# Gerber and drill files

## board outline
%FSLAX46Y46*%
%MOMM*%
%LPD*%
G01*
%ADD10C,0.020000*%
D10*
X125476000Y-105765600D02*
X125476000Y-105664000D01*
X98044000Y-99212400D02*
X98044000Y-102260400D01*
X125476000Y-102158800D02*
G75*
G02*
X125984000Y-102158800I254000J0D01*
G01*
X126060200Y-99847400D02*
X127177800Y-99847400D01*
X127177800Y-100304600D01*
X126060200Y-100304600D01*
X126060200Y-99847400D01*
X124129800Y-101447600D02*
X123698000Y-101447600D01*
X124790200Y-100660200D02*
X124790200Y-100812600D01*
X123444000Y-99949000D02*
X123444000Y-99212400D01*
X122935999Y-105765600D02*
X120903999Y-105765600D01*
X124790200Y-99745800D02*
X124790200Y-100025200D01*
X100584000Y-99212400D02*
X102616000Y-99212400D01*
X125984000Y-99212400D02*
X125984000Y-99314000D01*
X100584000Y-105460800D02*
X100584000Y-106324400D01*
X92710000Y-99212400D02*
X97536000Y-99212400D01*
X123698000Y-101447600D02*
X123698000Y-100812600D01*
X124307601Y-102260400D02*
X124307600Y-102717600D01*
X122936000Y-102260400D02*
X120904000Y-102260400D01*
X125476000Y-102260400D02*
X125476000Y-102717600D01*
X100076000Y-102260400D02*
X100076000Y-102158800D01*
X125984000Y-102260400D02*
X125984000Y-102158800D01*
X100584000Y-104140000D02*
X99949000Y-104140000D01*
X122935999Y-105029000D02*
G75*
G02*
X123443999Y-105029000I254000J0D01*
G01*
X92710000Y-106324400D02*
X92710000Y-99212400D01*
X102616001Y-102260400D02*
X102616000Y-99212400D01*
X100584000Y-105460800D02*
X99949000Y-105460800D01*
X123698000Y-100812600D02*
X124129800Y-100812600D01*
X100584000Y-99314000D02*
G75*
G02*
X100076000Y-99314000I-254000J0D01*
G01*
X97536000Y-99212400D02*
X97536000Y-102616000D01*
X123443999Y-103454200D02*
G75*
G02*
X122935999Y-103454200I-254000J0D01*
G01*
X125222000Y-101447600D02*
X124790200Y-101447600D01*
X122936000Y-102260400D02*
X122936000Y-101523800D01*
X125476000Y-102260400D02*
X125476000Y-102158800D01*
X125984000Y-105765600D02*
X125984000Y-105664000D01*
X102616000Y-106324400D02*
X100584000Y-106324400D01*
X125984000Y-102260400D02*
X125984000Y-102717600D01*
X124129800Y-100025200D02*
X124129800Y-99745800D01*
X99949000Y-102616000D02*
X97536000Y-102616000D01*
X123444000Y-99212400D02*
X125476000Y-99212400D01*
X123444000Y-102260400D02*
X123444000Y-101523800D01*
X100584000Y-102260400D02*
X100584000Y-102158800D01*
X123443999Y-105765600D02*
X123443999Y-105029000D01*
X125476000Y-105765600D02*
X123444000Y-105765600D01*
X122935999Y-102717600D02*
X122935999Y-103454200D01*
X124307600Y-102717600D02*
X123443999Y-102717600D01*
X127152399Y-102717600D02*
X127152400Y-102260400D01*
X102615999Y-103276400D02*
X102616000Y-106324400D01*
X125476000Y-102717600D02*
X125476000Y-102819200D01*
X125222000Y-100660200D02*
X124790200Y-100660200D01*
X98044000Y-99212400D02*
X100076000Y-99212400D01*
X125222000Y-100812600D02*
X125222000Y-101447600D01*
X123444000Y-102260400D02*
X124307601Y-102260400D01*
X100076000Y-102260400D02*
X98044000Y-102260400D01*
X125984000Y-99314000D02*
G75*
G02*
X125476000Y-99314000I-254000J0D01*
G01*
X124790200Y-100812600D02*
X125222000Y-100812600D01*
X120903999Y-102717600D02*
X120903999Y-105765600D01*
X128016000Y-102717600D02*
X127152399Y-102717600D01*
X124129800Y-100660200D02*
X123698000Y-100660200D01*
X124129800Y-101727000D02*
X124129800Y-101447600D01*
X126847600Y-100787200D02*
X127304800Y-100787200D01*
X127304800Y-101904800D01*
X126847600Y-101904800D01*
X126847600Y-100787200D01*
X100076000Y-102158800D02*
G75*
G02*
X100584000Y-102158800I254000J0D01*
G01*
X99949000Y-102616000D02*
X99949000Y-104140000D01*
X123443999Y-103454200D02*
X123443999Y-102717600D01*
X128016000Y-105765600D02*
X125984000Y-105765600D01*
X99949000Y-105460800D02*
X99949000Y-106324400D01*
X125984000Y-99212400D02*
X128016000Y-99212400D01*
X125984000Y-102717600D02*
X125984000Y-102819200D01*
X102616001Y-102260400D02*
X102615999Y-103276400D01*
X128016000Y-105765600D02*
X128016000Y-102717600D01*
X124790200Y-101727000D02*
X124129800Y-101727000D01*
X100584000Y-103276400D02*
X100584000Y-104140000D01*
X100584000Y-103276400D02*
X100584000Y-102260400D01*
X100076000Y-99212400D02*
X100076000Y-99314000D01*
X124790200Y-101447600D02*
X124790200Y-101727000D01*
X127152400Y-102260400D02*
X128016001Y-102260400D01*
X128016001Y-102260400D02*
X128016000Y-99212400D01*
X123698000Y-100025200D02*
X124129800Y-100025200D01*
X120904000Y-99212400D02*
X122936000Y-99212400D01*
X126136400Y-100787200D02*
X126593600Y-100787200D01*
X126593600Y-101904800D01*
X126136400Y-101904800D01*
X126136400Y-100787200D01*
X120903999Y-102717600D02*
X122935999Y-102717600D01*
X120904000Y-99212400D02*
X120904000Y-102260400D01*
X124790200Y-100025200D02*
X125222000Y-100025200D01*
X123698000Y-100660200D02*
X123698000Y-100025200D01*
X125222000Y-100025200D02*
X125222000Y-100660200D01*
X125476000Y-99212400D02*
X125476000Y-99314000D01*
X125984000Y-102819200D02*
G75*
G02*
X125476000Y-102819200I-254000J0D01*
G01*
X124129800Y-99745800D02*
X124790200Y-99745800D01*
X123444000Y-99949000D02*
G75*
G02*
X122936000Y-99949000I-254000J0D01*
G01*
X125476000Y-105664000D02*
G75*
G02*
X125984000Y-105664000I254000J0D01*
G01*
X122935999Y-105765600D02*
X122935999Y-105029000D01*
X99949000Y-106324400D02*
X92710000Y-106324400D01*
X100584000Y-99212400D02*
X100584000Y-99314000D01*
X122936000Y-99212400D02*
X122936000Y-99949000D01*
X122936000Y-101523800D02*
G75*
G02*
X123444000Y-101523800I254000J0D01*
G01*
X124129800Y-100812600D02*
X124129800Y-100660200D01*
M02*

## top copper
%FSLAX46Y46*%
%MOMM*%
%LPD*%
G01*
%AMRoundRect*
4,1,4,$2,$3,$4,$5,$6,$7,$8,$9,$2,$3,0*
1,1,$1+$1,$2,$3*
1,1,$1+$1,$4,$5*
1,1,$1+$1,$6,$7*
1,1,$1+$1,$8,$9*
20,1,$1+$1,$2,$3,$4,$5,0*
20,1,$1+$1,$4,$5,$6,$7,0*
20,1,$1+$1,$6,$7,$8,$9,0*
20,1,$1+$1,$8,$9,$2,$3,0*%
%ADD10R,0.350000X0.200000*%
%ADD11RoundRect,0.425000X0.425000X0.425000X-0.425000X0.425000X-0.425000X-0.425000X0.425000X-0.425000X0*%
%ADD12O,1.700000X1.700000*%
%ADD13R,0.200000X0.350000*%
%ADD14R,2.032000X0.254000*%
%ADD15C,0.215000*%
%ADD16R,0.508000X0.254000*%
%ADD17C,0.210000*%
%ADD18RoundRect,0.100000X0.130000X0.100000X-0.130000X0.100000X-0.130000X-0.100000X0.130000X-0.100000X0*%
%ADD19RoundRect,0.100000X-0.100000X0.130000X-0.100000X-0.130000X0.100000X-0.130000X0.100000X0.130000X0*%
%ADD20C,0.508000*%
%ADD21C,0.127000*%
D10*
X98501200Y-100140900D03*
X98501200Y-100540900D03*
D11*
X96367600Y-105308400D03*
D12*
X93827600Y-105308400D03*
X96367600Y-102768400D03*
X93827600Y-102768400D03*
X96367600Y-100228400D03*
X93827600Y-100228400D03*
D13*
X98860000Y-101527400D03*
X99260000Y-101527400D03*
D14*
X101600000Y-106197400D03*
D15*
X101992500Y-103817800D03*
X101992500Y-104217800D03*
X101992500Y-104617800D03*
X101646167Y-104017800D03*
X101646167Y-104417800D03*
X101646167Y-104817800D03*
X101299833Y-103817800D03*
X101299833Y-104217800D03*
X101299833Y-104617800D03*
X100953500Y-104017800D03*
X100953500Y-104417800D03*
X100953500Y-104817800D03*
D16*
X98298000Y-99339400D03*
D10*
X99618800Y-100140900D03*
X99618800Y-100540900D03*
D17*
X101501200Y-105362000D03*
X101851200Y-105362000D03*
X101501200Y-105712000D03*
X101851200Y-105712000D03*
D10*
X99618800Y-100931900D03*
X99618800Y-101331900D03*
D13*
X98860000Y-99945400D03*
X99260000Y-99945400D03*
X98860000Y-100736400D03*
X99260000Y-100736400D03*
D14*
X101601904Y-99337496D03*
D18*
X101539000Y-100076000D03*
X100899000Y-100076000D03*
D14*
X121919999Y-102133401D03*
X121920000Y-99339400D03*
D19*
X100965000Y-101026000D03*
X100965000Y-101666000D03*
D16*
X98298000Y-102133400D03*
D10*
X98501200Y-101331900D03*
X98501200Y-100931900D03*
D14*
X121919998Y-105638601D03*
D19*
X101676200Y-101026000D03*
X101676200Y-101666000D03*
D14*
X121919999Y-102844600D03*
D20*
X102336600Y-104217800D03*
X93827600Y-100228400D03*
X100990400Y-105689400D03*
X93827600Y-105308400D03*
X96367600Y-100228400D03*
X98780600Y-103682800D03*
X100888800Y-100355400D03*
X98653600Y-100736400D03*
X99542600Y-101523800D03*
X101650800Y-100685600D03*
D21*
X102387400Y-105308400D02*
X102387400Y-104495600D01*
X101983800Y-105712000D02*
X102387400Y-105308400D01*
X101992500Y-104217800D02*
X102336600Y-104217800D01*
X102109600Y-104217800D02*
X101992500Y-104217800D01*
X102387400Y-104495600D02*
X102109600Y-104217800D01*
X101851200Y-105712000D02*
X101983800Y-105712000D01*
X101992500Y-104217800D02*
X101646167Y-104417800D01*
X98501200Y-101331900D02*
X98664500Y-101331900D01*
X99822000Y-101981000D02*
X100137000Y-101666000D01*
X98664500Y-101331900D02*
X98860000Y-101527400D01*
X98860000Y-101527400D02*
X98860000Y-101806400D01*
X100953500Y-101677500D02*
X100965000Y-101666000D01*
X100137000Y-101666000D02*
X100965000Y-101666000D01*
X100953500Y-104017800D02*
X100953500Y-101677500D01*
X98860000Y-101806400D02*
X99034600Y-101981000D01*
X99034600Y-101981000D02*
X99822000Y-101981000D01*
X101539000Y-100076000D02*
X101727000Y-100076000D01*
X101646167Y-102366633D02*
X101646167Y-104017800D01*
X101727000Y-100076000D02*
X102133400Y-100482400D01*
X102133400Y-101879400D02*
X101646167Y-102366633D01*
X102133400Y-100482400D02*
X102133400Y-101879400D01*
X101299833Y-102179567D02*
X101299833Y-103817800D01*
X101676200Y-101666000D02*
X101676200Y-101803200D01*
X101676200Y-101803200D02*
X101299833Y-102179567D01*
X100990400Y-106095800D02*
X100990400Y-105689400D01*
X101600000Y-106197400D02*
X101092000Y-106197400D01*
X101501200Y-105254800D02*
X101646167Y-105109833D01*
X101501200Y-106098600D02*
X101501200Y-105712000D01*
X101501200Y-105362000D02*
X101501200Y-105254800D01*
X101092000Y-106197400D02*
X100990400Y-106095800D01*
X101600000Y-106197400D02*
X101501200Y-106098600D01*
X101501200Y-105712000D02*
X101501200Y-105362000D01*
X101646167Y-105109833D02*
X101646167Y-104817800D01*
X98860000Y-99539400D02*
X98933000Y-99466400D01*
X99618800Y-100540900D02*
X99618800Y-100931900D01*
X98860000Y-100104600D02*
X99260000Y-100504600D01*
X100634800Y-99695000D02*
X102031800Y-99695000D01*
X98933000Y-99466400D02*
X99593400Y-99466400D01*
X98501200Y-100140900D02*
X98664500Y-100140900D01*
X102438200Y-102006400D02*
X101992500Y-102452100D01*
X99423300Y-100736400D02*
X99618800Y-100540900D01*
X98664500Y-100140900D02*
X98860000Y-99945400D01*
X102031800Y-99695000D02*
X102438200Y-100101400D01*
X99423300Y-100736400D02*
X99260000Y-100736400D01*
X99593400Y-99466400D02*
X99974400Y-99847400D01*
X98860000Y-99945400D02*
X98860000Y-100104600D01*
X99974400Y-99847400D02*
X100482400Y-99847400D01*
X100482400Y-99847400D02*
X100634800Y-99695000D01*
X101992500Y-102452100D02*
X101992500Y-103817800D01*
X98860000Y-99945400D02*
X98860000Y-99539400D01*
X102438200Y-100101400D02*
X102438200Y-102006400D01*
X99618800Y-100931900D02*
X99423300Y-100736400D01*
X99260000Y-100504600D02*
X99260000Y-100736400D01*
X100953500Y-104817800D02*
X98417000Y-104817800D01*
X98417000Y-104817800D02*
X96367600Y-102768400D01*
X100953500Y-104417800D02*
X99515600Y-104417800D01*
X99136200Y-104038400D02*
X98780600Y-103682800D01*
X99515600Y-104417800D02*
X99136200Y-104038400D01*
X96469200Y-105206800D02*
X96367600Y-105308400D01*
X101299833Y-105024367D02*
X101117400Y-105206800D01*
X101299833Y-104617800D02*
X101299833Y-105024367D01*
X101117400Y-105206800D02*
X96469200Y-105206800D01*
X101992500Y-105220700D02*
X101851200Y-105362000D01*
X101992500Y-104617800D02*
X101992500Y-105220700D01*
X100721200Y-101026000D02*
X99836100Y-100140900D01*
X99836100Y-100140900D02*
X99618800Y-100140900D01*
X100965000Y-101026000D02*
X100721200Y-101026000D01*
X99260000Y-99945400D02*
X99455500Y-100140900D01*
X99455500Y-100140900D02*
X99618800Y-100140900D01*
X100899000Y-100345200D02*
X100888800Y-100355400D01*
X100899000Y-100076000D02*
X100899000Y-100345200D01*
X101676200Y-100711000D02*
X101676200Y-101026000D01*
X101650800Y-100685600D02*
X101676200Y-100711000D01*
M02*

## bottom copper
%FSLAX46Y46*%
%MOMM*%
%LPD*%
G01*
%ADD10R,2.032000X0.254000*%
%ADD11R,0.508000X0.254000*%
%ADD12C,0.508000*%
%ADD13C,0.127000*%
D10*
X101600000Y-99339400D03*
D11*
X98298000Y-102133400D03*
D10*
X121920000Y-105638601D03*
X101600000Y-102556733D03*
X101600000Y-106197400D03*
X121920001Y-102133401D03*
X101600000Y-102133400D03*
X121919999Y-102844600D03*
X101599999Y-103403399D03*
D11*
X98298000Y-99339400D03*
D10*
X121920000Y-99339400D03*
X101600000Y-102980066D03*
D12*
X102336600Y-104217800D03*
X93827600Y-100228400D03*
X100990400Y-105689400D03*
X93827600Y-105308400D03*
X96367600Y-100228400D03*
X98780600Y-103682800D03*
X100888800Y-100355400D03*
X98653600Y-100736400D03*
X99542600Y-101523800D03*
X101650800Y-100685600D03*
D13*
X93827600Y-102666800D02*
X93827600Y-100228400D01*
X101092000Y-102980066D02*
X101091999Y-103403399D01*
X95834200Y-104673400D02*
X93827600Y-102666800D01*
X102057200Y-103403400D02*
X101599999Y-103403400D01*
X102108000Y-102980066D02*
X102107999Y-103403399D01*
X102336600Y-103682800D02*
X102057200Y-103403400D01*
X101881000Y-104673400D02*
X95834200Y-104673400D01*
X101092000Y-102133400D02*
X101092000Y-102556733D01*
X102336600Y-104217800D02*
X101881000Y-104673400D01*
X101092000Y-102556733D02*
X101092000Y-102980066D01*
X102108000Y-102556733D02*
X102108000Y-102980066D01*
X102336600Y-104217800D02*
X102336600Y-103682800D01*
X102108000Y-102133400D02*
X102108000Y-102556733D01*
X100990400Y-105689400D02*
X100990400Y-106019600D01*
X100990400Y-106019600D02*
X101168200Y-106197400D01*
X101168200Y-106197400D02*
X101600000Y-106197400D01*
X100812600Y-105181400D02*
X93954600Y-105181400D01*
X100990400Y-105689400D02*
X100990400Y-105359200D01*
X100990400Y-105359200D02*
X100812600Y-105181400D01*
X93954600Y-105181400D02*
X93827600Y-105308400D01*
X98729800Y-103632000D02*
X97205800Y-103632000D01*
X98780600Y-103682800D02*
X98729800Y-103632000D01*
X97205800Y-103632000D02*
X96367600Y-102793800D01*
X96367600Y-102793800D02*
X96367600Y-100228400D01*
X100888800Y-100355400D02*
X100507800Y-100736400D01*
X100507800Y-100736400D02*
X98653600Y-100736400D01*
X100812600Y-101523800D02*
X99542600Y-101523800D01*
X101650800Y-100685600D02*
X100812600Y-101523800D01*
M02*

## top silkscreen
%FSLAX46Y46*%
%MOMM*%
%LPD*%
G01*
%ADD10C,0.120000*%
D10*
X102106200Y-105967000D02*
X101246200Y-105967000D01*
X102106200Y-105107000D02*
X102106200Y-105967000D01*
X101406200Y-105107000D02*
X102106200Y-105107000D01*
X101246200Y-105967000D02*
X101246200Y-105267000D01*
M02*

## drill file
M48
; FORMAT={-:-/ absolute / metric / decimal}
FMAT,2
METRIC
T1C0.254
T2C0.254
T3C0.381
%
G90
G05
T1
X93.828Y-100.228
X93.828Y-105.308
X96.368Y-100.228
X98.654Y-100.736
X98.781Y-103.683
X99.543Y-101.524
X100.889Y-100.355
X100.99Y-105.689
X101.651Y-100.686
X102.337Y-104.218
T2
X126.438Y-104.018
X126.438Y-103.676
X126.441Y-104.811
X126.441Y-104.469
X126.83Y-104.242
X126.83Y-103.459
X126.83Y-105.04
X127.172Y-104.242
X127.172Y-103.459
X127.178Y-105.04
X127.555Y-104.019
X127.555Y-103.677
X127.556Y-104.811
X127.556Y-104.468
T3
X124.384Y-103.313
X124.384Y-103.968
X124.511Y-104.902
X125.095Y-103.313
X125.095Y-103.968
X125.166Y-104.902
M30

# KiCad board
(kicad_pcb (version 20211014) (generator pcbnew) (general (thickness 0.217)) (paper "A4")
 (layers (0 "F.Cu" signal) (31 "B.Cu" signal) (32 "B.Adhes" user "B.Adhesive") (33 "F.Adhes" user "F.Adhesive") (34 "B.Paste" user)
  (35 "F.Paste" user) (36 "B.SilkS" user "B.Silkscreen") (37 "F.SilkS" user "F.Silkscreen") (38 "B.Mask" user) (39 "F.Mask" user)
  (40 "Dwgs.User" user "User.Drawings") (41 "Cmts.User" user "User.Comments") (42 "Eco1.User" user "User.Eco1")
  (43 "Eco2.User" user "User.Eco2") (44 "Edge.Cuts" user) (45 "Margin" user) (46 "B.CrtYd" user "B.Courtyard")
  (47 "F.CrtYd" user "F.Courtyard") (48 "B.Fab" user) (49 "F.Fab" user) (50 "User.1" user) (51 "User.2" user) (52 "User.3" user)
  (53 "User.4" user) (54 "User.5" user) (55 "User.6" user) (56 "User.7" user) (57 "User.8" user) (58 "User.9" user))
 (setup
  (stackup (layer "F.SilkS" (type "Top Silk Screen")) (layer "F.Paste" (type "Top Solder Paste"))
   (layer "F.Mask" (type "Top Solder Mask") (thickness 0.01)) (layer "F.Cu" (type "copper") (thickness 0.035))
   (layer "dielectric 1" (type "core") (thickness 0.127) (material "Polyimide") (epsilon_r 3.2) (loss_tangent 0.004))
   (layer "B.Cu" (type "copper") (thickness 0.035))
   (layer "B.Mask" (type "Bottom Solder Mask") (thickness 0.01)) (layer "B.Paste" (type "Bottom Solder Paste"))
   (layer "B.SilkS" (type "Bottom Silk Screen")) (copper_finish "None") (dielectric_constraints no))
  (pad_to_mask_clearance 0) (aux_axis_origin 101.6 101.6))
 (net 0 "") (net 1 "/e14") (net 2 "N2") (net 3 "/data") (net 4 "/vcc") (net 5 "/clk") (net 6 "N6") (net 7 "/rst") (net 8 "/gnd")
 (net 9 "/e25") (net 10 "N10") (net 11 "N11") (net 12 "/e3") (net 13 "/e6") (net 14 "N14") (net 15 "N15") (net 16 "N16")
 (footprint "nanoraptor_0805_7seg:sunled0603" (layer "F.Cu") (at 98.5012 100.3409 90)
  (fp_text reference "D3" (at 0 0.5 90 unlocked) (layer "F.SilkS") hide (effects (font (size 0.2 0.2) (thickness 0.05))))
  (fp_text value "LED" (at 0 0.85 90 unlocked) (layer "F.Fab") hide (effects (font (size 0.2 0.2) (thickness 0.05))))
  (pad "1" smd rect (at 0.2 0 90) (size 0.2 0.35) (layers "F.Cu" "F.Paste" "F.Mask") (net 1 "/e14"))
  (pad "2" smd rect (at -0.2 0 90) (size 0.2 0.35) (layers "F.Cu" "F.Paste" "F.Mask") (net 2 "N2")))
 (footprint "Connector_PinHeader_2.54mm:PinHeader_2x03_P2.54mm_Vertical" (layer "F.Cu") (at 95.0976 102.7684 180)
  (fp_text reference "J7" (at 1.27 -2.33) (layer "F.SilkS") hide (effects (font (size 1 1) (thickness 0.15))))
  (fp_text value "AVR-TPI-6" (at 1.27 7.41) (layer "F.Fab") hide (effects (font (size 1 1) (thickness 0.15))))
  (pad "1" smd roundrect (at -1.27 -2.54 180) (size 1.7 1.7) (layers "F.Cu" "F.Paste" "F.Mask") (roundrect_rratio 0.25) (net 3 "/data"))
  (pad "2" smd oval (at 1.27 -2.54 180) (size 1.7 1.7) (layers "F.Cu" "F.Paste" "F.Mask") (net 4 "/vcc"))
  (pad "3" smd oval (at -1.27 0 180) (size 1.7 1.7) (layers "F.Cu" "F.Paste" "F.Mask") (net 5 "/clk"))
  (pad "4" smd oval (at 1.27 0 180) (size 1.7 1.7) (layers "F.Cu" "F.Paste" "F.Mask") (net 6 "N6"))
  (pad "5" smd oval (at -1.27 2.54 180) (size 1.7 1.7) (layers "F.Cu" "F.Paste" "F.Mask") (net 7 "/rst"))
  (pad "6" smd oval (at 1.27 2.54 180) (size 1.7 1.7) (layers "F.Cu" "F.Paste" "F.Mask") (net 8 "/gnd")))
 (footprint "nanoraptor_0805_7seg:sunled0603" (layer "F.Cu") (at 99.06 101.5274 180)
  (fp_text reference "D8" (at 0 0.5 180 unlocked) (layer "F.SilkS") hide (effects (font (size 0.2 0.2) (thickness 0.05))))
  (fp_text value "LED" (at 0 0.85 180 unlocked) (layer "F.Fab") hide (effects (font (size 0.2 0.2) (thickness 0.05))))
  (pad "1" smd rect (at 0.2 0 180) (size 0.2 0.35) (layers "F.Cu" "F.Paste" "F.Mask") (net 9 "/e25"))
  (pad "2" smd rect (at -0.2 0 180) (size 0.2 0.35) (layers "F.Cu" "F.Paste" "F.Mask") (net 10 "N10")))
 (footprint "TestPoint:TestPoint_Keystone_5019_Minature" (layer "F.Cu") (at 101.6 106.1974)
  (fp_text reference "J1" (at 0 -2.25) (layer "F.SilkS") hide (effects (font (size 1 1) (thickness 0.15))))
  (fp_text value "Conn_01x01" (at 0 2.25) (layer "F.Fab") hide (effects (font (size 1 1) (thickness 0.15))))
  (pad "1" smd rect (at 0 0) (size 2.032 0.254) (layers "F.Cu" "F.Paste" "F.Mask") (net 4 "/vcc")))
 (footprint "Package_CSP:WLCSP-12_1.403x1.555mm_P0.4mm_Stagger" (layer "F.Cu") (at 101.473 104.3178 -90) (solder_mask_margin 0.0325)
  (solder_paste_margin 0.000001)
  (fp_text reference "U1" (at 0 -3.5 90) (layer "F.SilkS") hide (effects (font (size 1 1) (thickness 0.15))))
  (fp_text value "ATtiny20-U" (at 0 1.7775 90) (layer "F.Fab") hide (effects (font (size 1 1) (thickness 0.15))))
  (pad "A1" smd circle (at -0.5 -0.5195 270) (size 0.215 0.215) (layers "F.Cu" "F.Paste" "F.Mask") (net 1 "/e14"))
  (pad "A3" smd circle (at -0.1 -0.5195 270) (size 0.215 0.215) (layers "F.Cu" "F.Paste" "F.Mask") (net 8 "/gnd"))
  (pad "A5" smd circle (at 0.3 -0.5195 270) (size 0.215 0.215) (layers "F.Cu" "F.Paste" "F.Mask") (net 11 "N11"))
  (pad "B2" smd circle (at -0.3 -0.173167 270) (size 0.215 0.215) (layers "F.Cu" "F.Paste" "F.Mask") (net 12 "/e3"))
  (pad "B4" smd circle (at 0.1 -0.173167 270) (size 0.215 0.215) (layers "F.Cu" "F.Paste" "F.Mask") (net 8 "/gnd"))
  (pad "B6" smd circle (at 0.5 -0.173167 270) (size 0.215 0.215) (layers "F.Cu" "F.Paste" "F.Mask") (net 4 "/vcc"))
  (pad "C1" smd circle (at -0.5 0.173167 270) (size 0.215 0.215) (layers "F.Cu" "F.Paste" "F.Mask") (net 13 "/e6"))
  (pad "C3" smd circle (at -0.1 0.173167 270) (size 0.215 0.215) (layers "F.Cu" "F.Paste" "F.Mask") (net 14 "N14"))
  (pad "C5" smd circle (at 0.3 0.173167 270) (size 0.215 0.215) (layers "F.Cu" "F.Paste" "F.Mask") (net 3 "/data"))
  (pad "D2" smd circle (at -0.3 0.5195 270) (size 0.215 0.215) (layers "F.Cu" "F.Paste" "F.Mask") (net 9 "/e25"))
  (pad "D4" smd circle (at 0.1 0.5195 270) (size 0.215 0.215) (layers "F.Cu" "F.Paste" "F.Mask") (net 7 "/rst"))
  (pad "D6" smd circle (at 0.5 0.5195 270) (size 0.215 0.215) (layers "F.Cu" "F.Paste" "F.Mask") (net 5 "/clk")))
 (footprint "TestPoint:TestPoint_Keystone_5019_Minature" (layer "F.Cu") (at 98.298 99.3394)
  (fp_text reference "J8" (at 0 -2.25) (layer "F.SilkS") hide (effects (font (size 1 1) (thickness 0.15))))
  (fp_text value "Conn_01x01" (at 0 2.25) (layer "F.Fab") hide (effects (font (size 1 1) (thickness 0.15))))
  (pad "1" smd rect (at 0 0) (size 0.508 0.254) (layers "F.Cu" "F.Paste" "F.Mask")))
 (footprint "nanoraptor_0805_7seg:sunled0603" (layer "F.Cu") (at 99.6188 100.3409 90)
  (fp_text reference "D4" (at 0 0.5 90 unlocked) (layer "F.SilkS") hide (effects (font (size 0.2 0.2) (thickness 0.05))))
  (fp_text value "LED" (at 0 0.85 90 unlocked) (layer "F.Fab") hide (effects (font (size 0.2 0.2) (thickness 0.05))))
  (pad "1" smd rect (at 0.2 0 90) (size 0.2 0.35) (layers "F.Cu" "F.Paste" "F.Mask") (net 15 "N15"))
  (pad "2" smd rect (at -0.2 0 90) (size 0.2 0.35) (layers "F.Cu" "F.Paste" "F.Mask") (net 1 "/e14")))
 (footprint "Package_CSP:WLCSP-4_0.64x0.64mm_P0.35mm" (layer "F.Cu") (at 101.6762 105.537)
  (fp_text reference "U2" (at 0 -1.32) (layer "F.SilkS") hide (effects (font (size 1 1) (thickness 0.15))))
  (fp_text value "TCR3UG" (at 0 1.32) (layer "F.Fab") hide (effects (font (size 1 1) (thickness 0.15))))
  (fp_line (start 0.43 0.43) (end -0.43 0.43) (layer "F.SilkS") (width 0.12))
  (fp_line (start 0.43 -0.43) (end 0.43 0.43) (layer "F.SilkS") (width 0.12))
  (fp_line (start -0.27 -0.43) (end 0.43 -0.43) (layer "F.SilkS") (width 0.12))
  (fp_line (start -0.43 0.43) (end -0.43 -0.27) (layer "F.SilkS") (width 0.12))
  (pad "A1" smd circle (at -0.175 -0.175) (size 0.21 0.21) (layers "F.Cu" "F.Paste" "F.Mask") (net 4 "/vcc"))
  (pad "A2" smd circle (at 0.175 -0.175) (size 0.21 0.21) (layers "F.Cu" "F.Paste" "F.Mask") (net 11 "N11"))
  (pad "B1" smd circle (at -0.175 0.175) (size 0.21 0.21) (layers "F.Cu" "F.Paste" "F.Mask") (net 4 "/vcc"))
  (pad "B2" smd circle (at 0.175 0.175) (size 0.21 0.21) (layers "F.Cu" "F.Paste" "F.Mask") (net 8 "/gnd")))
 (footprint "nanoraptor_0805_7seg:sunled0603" (layer "F.Cu") (at 99.6188 101.1319 90)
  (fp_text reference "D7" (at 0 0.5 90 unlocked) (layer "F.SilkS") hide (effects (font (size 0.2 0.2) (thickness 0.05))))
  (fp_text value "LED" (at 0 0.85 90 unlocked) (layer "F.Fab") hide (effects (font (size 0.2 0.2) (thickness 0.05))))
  (pad "1" smd rect (at 0.2 0 90) (size 0.2 0.35) (layers "F.Cu" "F.Paste" "F.Mask") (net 1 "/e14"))
  (pad "2" smd rect (at -0.2 0 90) (size 0.2 0.35) (layers "F.Cu" "F.Paste" "F.Mask") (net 10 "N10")))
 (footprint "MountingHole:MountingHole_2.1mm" (layer "F.Cu") (at 131.699 105.0907 180)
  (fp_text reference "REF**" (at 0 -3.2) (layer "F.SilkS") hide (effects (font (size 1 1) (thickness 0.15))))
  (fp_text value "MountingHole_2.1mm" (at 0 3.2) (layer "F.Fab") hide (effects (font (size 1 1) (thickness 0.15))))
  (pad "" np_thru_hole circle (at 7.3152 1.778 270) (size 0.381 0.381) (drill 0.381) (layers F&B.Cu *.Mask))
  (pad "" np_thru_hole circle (at 7.1882 0.1887 180) (size 0.381 0.381) (drill 0.381) (layers F&B.Cu *.Mask))
  (pad "" np_thru_hole circle (at 4.527049 0.848616 270) (size 0.254 0.254) (drill 0.254) (layers F&B.Cu *.Mask))
  (pad "" np_thru_hole circle (at 5.2578 0.2794 180) (size 0.254 0.254) (drill 0.254) (layers F&B.Cu *.Mask))
  (pad "" np_thru_hole circle (at 5.257799 0.621841 180) (size 0.254 0.254) (drill 0.254) (layers F&B.Cu *.Mask))
  (pad "" np_thru_hole circle (at 7.315023 1.122827 270) (size 0.381 0.381) (drill 0.381) (layers F&B.Cu *.Mask))
  (pad "" np_thru_hole circle (at 4.142991 0.622581) (size 0.254 0.254) (drill 0.254) (layers F&B.Cu *.Mask))
  (pad "" np_thru_hole circle (at 4.142992 0.28014) (size 0.254 0.254) (drill 0.254) (layers F&B.Cu *.Mask))
  (pad "" np_thru_hole circle (at 6.603823 1.122827 270) (size 0.381 0.381) (drill 0.381) (layers F&B.Cu *.Mask))
  (pad "" np_thru_hole circle (at 5.261123 1.414676 180) (size 0.254 0.254) (drill 0.254) (layers F&B.Cu *.Mask))
  (pad "" np_thru_hole circle (at 5.261124 1.072235 180) (size 0.254 0.254) (drill 0.254) (layers F&B.Cu *.Mask))
  (pad "" np_thru_hole circle (at 4.143859 1.413906) (size 0.254 0.254) (drill 0.254) (layers F&B.Cu *.Mask))
  (pad "" np_thru_hole circle (at 4.869352 1.632031 90) (size 0.254 0.254) (drill 0.254) (layers F&B.Cu *.Mask))
  (pad "" np_thru_hole circle (at 4.86949 0.848617 270) (size 0.254 0.254) (drill 0.254) (layers F&B.Cu *.Mask))
  (pad "" np_thru_hole circle (at 6.604 1.778 270) (size 0.381 0.381) (drill 0.381) (layers F&B.Cu *.Mask))
  (pad "" np_thru_hole circle (at 4.526911 1.63203 90) (size 0.254 0.254) (drill 0.254) (layers F&B.Cu *.Mask))
  (pad "" np_thru_hole circle (at 4.14386 1.071465) (size 0.254 0.254) (drill 0.254) (layers F&B.Cu *.Mask))
  (pad "" np_thru_hole circle (at 4.5212 0.0508 180) (size 0.254 0.254) (drill 0.254) (layers F&B.Cu *.Mask))
  (pad "" np_thru_hole circle (at 6.533027 0.188877 180) (size 0.381 0.381) (drill 0.381) (layers F&B.Cu *.Mask))
  (pad "" np_thru_hole circle (at 4.868698 0.051155 180) (size 0.254 0.254) (drill 0.254) (layers F&B.Cu *.Mask)))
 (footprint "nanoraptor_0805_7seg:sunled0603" (layer "F.Cu") (at 99.06 99.9454 180)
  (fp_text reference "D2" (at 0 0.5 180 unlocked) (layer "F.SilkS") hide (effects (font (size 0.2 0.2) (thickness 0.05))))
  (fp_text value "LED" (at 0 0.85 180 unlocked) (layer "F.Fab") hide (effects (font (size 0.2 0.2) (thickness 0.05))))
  (pad "1" smd rect (at 0.2 0 180) (size 0.2 0.35) (layers "F.Cu" "F.Paste" "F.Mask") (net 1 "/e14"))
  (pad "2" smd rect (at -0.2 0 180) (size 0.2 0.35) (layers "F.Cu" "F.Paste" "F.Mask") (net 15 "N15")))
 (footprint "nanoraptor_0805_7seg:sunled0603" (layer "F.Cu") (at 99.06 100.7364 180)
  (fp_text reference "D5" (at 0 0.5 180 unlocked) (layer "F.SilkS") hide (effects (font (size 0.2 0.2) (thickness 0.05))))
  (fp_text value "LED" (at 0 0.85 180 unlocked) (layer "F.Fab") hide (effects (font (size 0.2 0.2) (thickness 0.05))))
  (pad "1" smd rect (at 0.2 0 180) (size 0.2 0.35) (layers "F.Cu" "F.Paste" "F.Mask") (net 2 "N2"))
  (pad "2" smd rect (at -0.2 0 180) (size 0.2 0.35) (layers "F.Cu" "F.Paste" "F.Mask") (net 1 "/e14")))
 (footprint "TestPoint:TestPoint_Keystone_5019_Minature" (layer "F.Cu") (at 101.6 99.3394 180)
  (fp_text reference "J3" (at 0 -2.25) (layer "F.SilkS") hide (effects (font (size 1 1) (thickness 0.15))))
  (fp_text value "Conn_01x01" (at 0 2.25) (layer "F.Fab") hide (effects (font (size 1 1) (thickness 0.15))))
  (pad "1" smd rect (at 0 0 180) (size 2.032 0.254) (layers "B.Cu" "B.Paste" "B.Mask") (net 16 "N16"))
  (pad "1" smd rect (at -0.001904 0.001904 180) (size 2.032 0.254) (layers "F.Cu" "F.Paste" "F.Mask") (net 16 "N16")))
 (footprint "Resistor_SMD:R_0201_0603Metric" (layer "F.Cu") (at 101.219 100.076 180)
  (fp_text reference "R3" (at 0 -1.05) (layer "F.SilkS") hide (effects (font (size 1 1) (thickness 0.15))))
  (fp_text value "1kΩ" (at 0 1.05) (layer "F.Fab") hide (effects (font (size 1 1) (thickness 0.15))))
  (pad "" smd roundrect (at -0.345 0 180) (size 0.318 0.36) (layers "F.Paste") (roundrect_rratio 0.25))
  (pad "" smd roundrect (at 0.345 0 180) (size 0.318 0.36) (layers "F.Paste") (roundrect_rratio 0.25))
  (pad "1" smd roundrect (at -0.32 0 180) (size 0.46 0.4) (layers "F.Cu" "F.Mask") (roundrect_rratio 0.25) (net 12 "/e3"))
  (pad "2" smd roundrect (at 0.32 0 180) (size 0.46 0.4) (layers "F.Cu" "F.Mask") (roundrect_rratio 0.25) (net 2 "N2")))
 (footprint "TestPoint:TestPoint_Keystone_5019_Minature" (layer "F.Cu") (at 121.919999 102.133401)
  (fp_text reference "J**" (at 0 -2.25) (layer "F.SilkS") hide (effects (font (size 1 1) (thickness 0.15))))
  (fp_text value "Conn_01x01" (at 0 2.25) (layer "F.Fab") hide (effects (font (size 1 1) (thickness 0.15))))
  (pad "1" smd rect (at 0 0) (size 2.032 0.254) (layers "F.Cu" "F.Paste" "F.Mask")))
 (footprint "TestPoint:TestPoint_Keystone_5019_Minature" (layer "F.Cu") (at 121.92 99.3394)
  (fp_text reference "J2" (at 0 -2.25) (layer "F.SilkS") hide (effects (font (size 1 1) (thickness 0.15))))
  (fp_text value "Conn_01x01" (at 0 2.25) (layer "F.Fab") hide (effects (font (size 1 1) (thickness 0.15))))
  (pad "1" smd rect (at 0 0) (size 2.032 0.254) (layers "F.Cu" "F.Paste" "F.Mask")))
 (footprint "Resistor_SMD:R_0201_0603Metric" (layer "F.Cu") (at 100.965 101.346 -90)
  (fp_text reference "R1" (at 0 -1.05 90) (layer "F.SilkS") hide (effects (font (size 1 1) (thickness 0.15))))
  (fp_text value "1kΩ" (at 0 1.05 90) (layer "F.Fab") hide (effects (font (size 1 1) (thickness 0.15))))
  (pad "" smd roundrect (at -0.345 0 270) (size 0.318 0.36) (layers "F.Paste") (roundrect_rratio 0.25))
  (pad "" smd roundrect (at 0.345 0 270) (size 0.318 0.36) (layers "F.Paste") (roundrect_rratio 0.25))
  (pad "1" smd roundrect (at -0.32 0 270) (size 0.46 0.4) (layers "F.Cu" "F.Mask") (roundrect_rratio 0.25) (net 15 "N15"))
  (pad "2" smd roundrect (at 0.32 0 270) (size 0.46 0.4) (layers "F.Cu" "F.Mask") (roundrect_rratio 0.25) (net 9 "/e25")))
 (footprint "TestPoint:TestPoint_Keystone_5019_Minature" (layer "F.Cu") (at 98.298 102.1334)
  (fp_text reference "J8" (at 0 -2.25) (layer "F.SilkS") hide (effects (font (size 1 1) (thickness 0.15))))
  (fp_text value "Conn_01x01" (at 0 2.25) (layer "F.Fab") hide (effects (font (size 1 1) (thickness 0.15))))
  (pad "1" smd rect (at 0 0) (size 0.508 0.254) (layers "F.Cu" "F.Paste" "F.Mask")))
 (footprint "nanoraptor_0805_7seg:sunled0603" (layer "F.Cu") (at 98.5012 101.1319 -90)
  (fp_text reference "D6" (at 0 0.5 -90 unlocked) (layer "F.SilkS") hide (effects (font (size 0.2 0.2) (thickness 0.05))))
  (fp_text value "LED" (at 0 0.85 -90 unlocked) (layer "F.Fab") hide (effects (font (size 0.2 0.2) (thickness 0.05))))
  (pad "1" smd rect (at 0.2 0 270) (size 0.2 0.35) (layers "F.Cu" "F.Paste" "F.Mask") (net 9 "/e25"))
  (pad "2" smd rect (at -0.2 0 270) (size 0.2 0.35) (layers "F.Cu" "F.Paste" "F.Mask") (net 2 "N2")))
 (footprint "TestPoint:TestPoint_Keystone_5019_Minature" (layer "F.Cu") (at 121.919998 105.638601)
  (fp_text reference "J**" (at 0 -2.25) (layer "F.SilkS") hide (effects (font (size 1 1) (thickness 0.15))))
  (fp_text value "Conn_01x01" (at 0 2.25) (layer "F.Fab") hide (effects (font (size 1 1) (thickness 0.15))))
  (pad "1" smd rect (at 0 0) (size 2.032 0.254) (layers "F.Cu" "F.Paste" "F.Mask")))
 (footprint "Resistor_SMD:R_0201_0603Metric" (layer "F.Cu") (at 101.6762 101.346 -90)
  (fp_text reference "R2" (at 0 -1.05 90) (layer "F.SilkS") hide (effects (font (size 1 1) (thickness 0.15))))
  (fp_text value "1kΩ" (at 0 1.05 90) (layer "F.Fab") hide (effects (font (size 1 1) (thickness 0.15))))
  (pad "" smd roundrect (at -0.345 0 270) (size 0.318 0.36) (layers "F.Paste") (roundrect_rratio 0.25))
  (pad "" smd roundrect (at 0.345 0 270) (size 0.318 0.36) (layers "F.Paste") (roundrect_rratio 0.25))
  (pad "1" smd roundrect (at -0.32 0 270) (size 0.46 0.4) (layers "F.Cu" "F.Mask") (roundrect_rratio 0.25) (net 10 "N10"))
  (pad "2" smd roundrect (at 0.32 0 270) (size 0.46 0.4) (layers "F.Cu" "F.Mask") (roundrect_rratio 0.25) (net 13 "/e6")))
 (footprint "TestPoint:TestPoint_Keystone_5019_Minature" (layer "F.Cu") (at 121.919999 102.8446)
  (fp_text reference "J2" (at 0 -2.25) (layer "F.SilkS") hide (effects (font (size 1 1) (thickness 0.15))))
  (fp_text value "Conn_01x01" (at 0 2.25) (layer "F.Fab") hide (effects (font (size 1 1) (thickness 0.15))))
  (pad "1" smd rect (at 0 0) (size 2.032 0.254) (layers "F.Cu" "F.Paste" "F.Mask")))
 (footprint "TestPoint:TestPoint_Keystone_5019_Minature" (layer "B.Cu") (at 98.298 102.1334 180)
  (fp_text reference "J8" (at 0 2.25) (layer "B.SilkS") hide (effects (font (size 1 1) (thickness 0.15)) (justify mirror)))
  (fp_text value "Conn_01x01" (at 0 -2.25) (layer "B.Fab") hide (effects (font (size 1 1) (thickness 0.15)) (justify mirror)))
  (pad "1" smd rect (at 0 0 180) (size 0.508 0.254) (layers "B.Cu" "B.Paste" "B.Mask")))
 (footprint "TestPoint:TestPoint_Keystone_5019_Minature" (layer "B.Cu") (at 121.92 105.638601 180)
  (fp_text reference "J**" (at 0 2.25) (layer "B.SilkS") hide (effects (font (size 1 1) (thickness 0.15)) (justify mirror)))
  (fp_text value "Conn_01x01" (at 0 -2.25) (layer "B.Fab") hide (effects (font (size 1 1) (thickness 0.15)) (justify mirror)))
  (pad "1" smd rect (at 0 0 180) (size 2.032 0.254) (layers "B.Cu" "B.Paste" "B.Mask")))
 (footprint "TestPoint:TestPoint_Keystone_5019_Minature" (layer "B.Cu") (at 101.6 102.556733 180)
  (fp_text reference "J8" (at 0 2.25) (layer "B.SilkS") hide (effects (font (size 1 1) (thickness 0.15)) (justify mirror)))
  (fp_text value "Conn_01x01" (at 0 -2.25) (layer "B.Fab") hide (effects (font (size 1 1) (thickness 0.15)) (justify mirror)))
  (pad "1" smd rect (at 0 0 180) (size 2.032 0.254) (layers "B.Cu" "B.Paste" "B.Mask") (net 8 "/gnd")))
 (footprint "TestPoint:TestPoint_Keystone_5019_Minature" (layer "B.Cu") (at 101.6 106.1974 180)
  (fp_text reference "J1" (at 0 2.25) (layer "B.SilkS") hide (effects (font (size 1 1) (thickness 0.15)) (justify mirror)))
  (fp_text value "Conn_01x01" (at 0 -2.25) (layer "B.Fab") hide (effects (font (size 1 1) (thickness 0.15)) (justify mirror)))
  (pad "1" smd rect (at 0 0 180) (size 2.032 0.254) (layers "B.Cu" "B.Paste" "B.Mask") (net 4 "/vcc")))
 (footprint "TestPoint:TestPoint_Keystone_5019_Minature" (layer "B.Cu") (at 121.920001 102.133401 180)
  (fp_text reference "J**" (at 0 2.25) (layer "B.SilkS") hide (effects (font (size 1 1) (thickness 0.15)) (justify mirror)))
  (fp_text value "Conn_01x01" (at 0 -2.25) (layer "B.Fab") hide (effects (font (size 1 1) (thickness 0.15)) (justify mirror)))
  (pad "1" smd rect (at 0 0 180) (size 2.032 0.254) (layers "B.Cu" "B.Paste" "B.Mask")))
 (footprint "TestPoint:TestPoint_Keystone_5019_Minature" (layer "B.Cu") (at 101.6 102.1334)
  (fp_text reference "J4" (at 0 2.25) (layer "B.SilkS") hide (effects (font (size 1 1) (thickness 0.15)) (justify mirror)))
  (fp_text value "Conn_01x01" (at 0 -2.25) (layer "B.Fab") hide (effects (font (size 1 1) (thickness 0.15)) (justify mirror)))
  (pad "1" smd rect (at 0 0) (size 2.032 0.254) (layers "B.Cu" "B.Paste" "B.Mask") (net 8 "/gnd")))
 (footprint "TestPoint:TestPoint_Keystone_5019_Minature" (layer "B.Cu") (at 121.919999 102.8446 180)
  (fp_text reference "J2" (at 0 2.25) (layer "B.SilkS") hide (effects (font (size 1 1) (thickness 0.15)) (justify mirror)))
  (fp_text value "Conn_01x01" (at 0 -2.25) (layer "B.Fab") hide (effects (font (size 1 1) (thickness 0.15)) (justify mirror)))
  (pad "1" smd rect (at 0 0 180) (size 2.032 0.254) (layers "B.Cu" "B.Paste" "B.Mask")))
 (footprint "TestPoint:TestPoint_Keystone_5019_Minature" (layer "B.Cu") (at 101.599999 103.403399 180)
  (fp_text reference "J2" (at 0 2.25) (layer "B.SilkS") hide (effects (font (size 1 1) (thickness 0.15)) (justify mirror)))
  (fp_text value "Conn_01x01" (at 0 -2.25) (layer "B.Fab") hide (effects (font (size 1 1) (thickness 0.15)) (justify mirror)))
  (pad "1" smd rect (at 0 0 180) (size 2.032 0.254) (layers "B.Cu" "B.Paste" "B.Mask") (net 8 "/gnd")))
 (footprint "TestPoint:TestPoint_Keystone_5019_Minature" (layer "B.Cu") (at 98.298 99.3394 180)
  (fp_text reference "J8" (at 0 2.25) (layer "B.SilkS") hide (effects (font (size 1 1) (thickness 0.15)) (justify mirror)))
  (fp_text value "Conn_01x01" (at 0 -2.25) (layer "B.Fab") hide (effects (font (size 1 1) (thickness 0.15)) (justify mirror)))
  (pad "1" smd rect (at 0 0 180) (size 0.508 0.254) (layers "B.Cu" "B.Paste" "B.Mask")))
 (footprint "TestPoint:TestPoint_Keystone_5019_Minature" (layer "B.Cu") (at 121.92 99.3394 180)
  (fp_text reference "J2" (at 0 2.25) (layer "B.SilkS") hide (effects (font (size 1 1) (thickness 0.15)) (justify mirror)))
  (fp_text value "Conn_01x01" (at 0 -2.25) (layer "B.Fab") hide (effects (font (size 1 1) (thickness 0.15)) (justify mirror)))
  (pad "1" smd rect (at 0 0 180) (size 2.032 0.254) (layers "B.Cu" "B.Paste" "B.Mask")))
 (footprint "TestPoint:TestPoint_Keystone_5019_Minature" (layer "B.Cu") (at 101.6 102.980066 180)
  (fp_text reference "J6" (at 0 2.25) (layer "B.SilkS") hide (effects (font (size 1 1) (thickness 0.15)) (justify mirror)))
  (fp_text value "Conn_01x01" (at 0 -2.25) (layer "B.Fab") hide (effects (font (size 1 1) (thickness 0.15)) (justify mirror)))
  (pad "1" smd rect (at 0 0 180) (size 2.032 0.254) (layers "B.Cu" "B.Paste" "B.Mask") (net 8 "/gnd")))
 (gr_line (start 125.476 105.7656) (end 125.476 105.664) (layer "Edge.Cuts") (width 0.02))
 (gr_line (start 98.044 99.2124) (end 98.044 102.2604) (layer "Edge.Cuts") (width 0.02))
 (gr_arc (start 125.476 102.1588) (mid 125.73 101.9048) (end 125.984 102.1588) (layer "Edge.Cuts") (width 0.02))
 (gr_rect (start 126.0602 99.8474) (end 127.1778 100.3046) (layer "Edge.Cuts") (width 0.02) (fill none))
 (gr_line (start 124.1298 101.4476) (end 123.698 101.4476) (layer "Edge.Cuts") (width 0.02))
 (gr_line (start 124.7902 100.6602) (end 124.7902 100.8126) (layer "Edge.Cuts") (width 0.02))
 (gr_line (start 123.444 99.949) (end 123.444 99.2124) (layer "Edge.Cuts") (width 0.02))
 (gr_line (start 122.935999 105.7656) (end 120.903999 105.7656) (layer "Edge.Cuts") (width 0.02))
 (gr_line (start 124.7902 99.7458) (end 124.7902 100.0252) (layer "Edge.Cuts") (width 0.02))
 (gr_line (start 100.584 99.2124) (end 102.616 99.2124) (layer "Edge.Cuts") (width 0.02))
 (gr_line (start 125.984 99.2124) (end 125.984 99.314) (layer "Edge.Cuts") (width 0.02))
 (gr_line (start 100.584 105.4608) (end 100.584 106.3244) (layer "Edge.Cuts") (width 0.02))
 (gr_line (start 92.71 99.2124) (end 97.536 99.2124) (layer "Edge.Cuts") (width 0.02))
 (gr_line (start 123.698 101.4476) (end 123.698 100.8126) (layer "Edge.Cuts") (width 0.02))
 (gr_line (start 124.307601 102.2604) (end 124.3076 102.7176) (layer "Edge.Cuts") (width 0.02))
 (gr_line (start 122.936 102.2604) (end 120.904 102.2604) (layer "Edge.Cuts") (width 0.02))
 (gr_line (start 125.476 102.2604) (end 125.476 102.7176) (layer "Edge.Cuts") (width 0.02))
 (gr_line (start 100.076 102.2604) (end 100.076 102.1588) (layer "Edge.Cuts") (width 0.02))
 (gr_line (start 125.984 102.2604) (end 125.984 102.1588) (layer "Edge.Cuts") (width 0.02))
 (gr_line (start 100.584 104.14) (end 99.949 104.14) (layer "Edge.Cuts") (width 0.02))
 (gr_arc (start 122.935999 105.029) (mid 123.189999 104.775) (end 123.443999 105.029) (layer "Edge.Cuts") (width 0.02))
 (gr_line (start 92.71 106.3244) (end 92.71 99.2124) (layer "Edge.Cuts") (width 0.02))
 (gr_line (start 102.616001 102.2604) (end 102.616 99.2124) (layer "Edge.Cuts") (width 0.02))
 (gr_line (start 100.584 105.4608) (end 99.949 105.4608) (layer "Edge.Cuts") (width 0.02))
 (gr_line (start 123.698 100.8126) (end 124.1298 100.8126) (layer "Edge.Cuts") (width 0.02))
 (gr_arc (start 100.584 99.314) (mid 100.33 99.568) (end 100.076 99.314) (layer "Edge.Cuts") (width 0.02))
 (gr_line (start 97.536 99.2124) (end 97.536 102.616) (layer "Edge.Cuts") (width 0.02))
 (gr_arc (start 123.443999 103.4542) (mid 123.189999 103.7082) (end 122.935999 103.4542) (layer "Edge.Cuts") (width 0.02))
 (gr_line (start 125.222 101.4476) (end 124.7902 101.4476) (layer "Edge.Cuts") (width 0.02))
 (gr_line (start 122.936 102.2604) (end 122.936 101.5238) (layer "Edge.Cuts") (width 0.02))
 (gr_line (start 125.476 102.2604) (end 125.476 102.1588) (layer "Edge.Cuts") (width 0.02))
 (gr_line (start 125.984 105.7656) (end 125.984 105.664) (layer "Edge.Cuts") (width 0.02))
 (gr_line (start 102.616 106.3244) (end 100.584 106.3244) (layer "Edge.Cuts") (width 0.02))
 (gr_line (start 125.984 102.2604) (end 125.984 102.7176) (layer "Edge.Cuts") (width 0.02))
 (gr_line (start 124.1298 100.0252) (end 124.1298 99.7458) (layer "Edge.Cuts") (width 0.02))
 (gr_line (start 99.949 102.616) (end 97.536 102.616) (layer "Edge.Cuts") (width 0.02))
 (gr_line (start 123.444 99.2124) (end 125.476 99.2124) (layer "Edge.Cuts") (width 0.02))
 (gr_line (start 123.444 102.2604) (end 123.444 101.5238) (layer "Edge.Cuts") (width 0.02))
 (gr_line (start 100.584 102.2604) (end 100.584 102.1588) (layer "Edge.Cuts") (width 0.02))
 (gr_line (start 123.443999 105.7656) (end 123.443999 105.029) (layer "Edge.Cuts") (width 0.02))
 (gr_line (start 125.476 105.7656) (end 123.444 105.7656) (layer "Edge.Cuts") (width 0.02))
 (gr_line (start 122.935999 102.7176) (end 122.935999 103.4542) (layer "Edge.Cuts") (width 0.02))
 (gr_line (start 124.3076 102.7176) (end 123.443999 102.7176) (layer "Edge.Cuts") (width 0.02))
 (gr_line (start 127.152399 102.7176) (end 127.1524 102.2604) (layer "Edge.Cuts") (width 0.02))
 (gr_line (start 102.615999 103.2764) (end 102.616 106.3244) (layer "Edge.Cuts") (width 0.02))
 (gr_line (start 125.476 102.7176) (end 125.476 102.8192) (layer "Edge.Cuts") (width 0.02))
 (gr_line (start 125.222 100.6602) (end 124.7902 100.6602) (layer "Edge.Cuts") (width 0.02))
 (gr_line (start 98.044 99.2124) (end 100.076 99.2124) (layer "Edge.Cuts") (width 0.02))
 (gr_line (start 125.222 100.8126) (end 125.222 101.4476) (layer "Edge.Cuts") (width 0.02))
 (gr_line (start 123.444 102.2604) (end 124.307601 102.2604) (layer "Edge.Cuts") (width 0.02))
 (gr_line (start 100.076 102.2604) (end 98.044 102.2604) (layer "Edge.Cuts") (width 0.02))
 (gr_arc (start 125.984 99.314) (mid 125.73 99.568) (end 125.476 99.314) (layer "Edge.Cuts") (width 0.02))
 (gr_line (start 124.7902 100.8126) (end 125.222 100.8126) (layer "Edge.Cuts") (width 0.02))
 (gr_line (start 120.903999 102.7176) (end 120.903999 105.7656) (layer "Edge.Cuts") (width 0.02))
 (gr_line (start 128.016 102.7176) (end 127.152399 102.7176) (layer "Edge.Cuts") (width 0.02))
 (gr_line (start 124.1298 100.6602) (end 123.698 100.6602) (layer "Edge.Cuts") (width 0.02))
 (gr_line (start 124.1298 101.727) (end 124.1298 101.4476) (layer "Edge.Cuts") (width 0.02))
 (gr_rect (start 126.8476 100.7872) (end 127.3048 101.9048) (layer "Edge.Cuts") (width 0.02) (fill none))
 (gr_arc (start 100.076 102.1588) (mid 100.33 101.9048) (end 100.584 102.1588) (layer "Edge.Cuts") (width 0.02))
 (gr_line (start 99.949 102.616) (end 99.949 104.14) (layer "Edge.Cuts") (width 0.02))
 (gr_line (start 123.443999 103.4542) (end 123.443999 102.7176) (layer "Edge.Cuts") (width 0.02))
 (gr_line (start 128.016 105.7656) (end 125.984 105.7656) (layer "Edge.Cuts") (width 0.02))
 (gr_line (start 99.949 105.4608) (end 99.949 106.3244) (layer "Edge.Cuts") (width 0.02))
 (gr_line (start 125.984 99.2124) (end 128.016 99.2124) (layer "Edge.Cuts") (width 0.02))
 (gr_line (start 125.984 102.7176) (end 125.984 102.8192) (layer "Edge.Cuts") (width 0.02))
 (gr_line (start 102.616001 102.2604) (end 102.615999 103.2764) (layer "Edge.Cuts") (width 0.02))
 (gr_line (start 128.016 105.7656) (end 128.016 102.7176) (layer "Edge.Cuts") (width 0.02))
 (gr_line (start 124.7902 101.727) (end 124.1298 101.727) (layer "Edge.Cuts") (width 0.02))
 (gr_line (start 100.584 103.2764) (end 100.584 104.14) (layer "Edge.Cuts") (width 0.02))
 (gr_line (start 100.584 103.2764) (end 100.584 102.2604) (layer "Edge.Cuts") (width 0.02))
 (gr_line (start 100.076 99.2124) (end 100.076 99.314) (layer "Edge.Cuts") (width 0.02))
 (gr_line (start 124.7902 101.4476) (end 124.7902 101.727) (layer "Edge.Cuts") (width 0.02))
 (gr_line (start 127.1524 102.2604) (end 128.016001 102.2604) (layer "Edge.Cuts") (width 0.02))
 (gr_line (start 128.016001 102.2604) (end 128.016 99.2124) (layer "Edge.Cuts") (width 0.02))
 (gr_line (start 123.698 100.0252) (end 124.1298 100.0252) (layer "Edge.Cuts") (width 0.02))
 (gr_line (start 120.904 99.2124) (end 122.936 99.2124) (layer "Edge.Cuts") (width 0.02))
 (gr_rect (start 126.1364 100.7872) (end 126.5936 101.9048) (layer "Edge.Cuts") (width 0.02) (fill none))
 (gr_line (start 120.903999 102.7176) (end 122.935999 102.7176) (layer "Edge.Cuts") (width 0.02))
 (gr_line (start 120.904 99.2124) (end 120.904 102.2604) (layer "Edge.Cuts") (width 0.02))
 (gr_line (start 124.7902 100.0252) (end 125.222 100.0252) (layer "Edge.Cuts") (width 0.02))
 (gr_line (start 123.698 100.6602) (end 123.698 100.0252) (layer "Edge.Cuts") (width 0.02))
 (gr_line (start 125.222 100.0252) (end 125.222 100.6602) (layer "Edge.Cuts") (width 0.02))
 (gr_line (start 125.476 99.2124) (end 125.476 99.314) (layer "Edge.Cuts") (width 0.02))
 (gr_arc (start 125.984 102.8192) (mid 125.73 103.0732) (end 125.476 102.8192) (layer "Edge.Cuts") (width 0.02))
 (gr_line (start 124.1298 99.7458) (end 124.7902 99.7458) (layer "Edge.Cuts") (width 0.02))
 (gr_arc (start 123.444 99.949) (mid 123.19 100.203) (end 122.936 99.949) (layer "Edge.Cuts") (width 0.02))
 (gr_arc (start 125.476 105.664) (mid 125.73 105.41) (end 125.984 105.664) (layer "Edge.Cuts") (width 0.02))
 (gr_line (start 122.935999 105.7656) (end 122.935999 105.029) (layer "Edge.Cuts") (width 0.02))
 (gr_line (start 99.949 106.3244) (end 92.71 106.3244) (layer "Edge.Cuts") (width 0.02))
 (gr_line (start 100.584 99.2124) (end 100.584 99.314) (layer "Edge.Cuts") (width 0.02))
 (gr_line (start 122.936 99.2124) (end 122.936 99.949) (layer "Edge.Cuts") (width 0.02))
 (gr_arc (start 122.936 101.5238) (mid 123.19 101.2698) (end 123.444 101.5238) (layer "Edge.Cuts") (width 0.02))
 (gr_line (start 124.1298 100.8126) (end 124.1298 100.6602) (layer "Edge.Cuts") (width 0.02))
 (segment (start 102.3874 105.3084) (end 102.3874 104.4956) (width 0.127) (layer "F.Cu") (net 8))
 (segment (start 101.9838 105.712) (end 102.3874 105.3084) (width 0.127) (layer "F.Cu") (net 8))
 (segment (start 101.9925 104.2178) (end 102.3366 104.2178) (width 0.127) (layer "F.Cu") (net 8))
 (segment (start 102.1096 104.2178) (end 101.9925 104.2178) (width 0.127) (layer "F.Cu") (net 8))
 (segment (start 102.3874 104.4956) (end 102.1096 104.2178) (width 0.127) (layer "F.Cu") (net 8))
 (segment (start 101.8512 105.712) (end 101.9838 105.712) (width 0.127) (layer "F.Cu") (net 8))
 (segment (start 101.9925 104.2178) (end 101.646167 104.4178) (width 0.127) (layer "F.Cu") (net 8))
 (via (at 102.3366 104.2178) (size 0.508) (drill 0.254) (layers "F.Cu" "B.Cu") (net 8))
 (via (at 93.8276 100.2284) (size 0.508) (drill 0.254) (layers "F.Cu" "B.Cu") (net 8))
 (segment (start 93.8276 102.6668) (end 93.8276 100.2284) (width 0.127) (layer "B.Cu") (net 8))
 (segment (start 101.092 102.980066) (end 101.091999 103.403399) (width 0.127) (layer "B.Cu") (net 8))
 (segment (start 95.8342 104.6734) (end 93.8276 102.6668) (width 0.127) (layer "B.Cu") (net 8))
 (segment (start 102.0572 103.4034) (end 101.599999 103.4034) (width 0.127) (layer "B.Cu") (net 8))
 (segment (start 102.108 102.980066) (end 102.107999 103.403399) (width 0.127) (layer "B.Cu") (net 8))
 (segment (start 102.3366 103.6828) (end 102.0572 103.4034) (width 0.127) (layer "B.Cu") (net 8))
 (segment (start 101.881 104.6734) (end 95.8342 104.6734) (width 0.127) (layer "B.Cu") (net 8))
 (segment (start 101.092 102.1334) (end 101.092 102.556733) (width 0.127) (layer "B.Cu") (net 8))
 (segment (start 102.3366 104.2178) (end 101.881 104.6734) (width 0.127) (layer "B.Cu") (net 8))
 (segment (start 101.092 102.556733) (end 101.092 102.980066) (width 0.127) (layer "B.Cu") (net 8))
 (segment (start 102.108 102.556733) (end 102.108 102.980066) (width 0.127) (layer "B.Cu") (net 8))
 (segment (start 102.3366 104.2178) (end 102.3366 103.6828) (width 0.127) (layer "B.Cu") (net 8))
 (segment (start 102.108 102.1334) (end 102.108 102.556733) (width 0.127) (layer "B.Cu") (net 8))
 (segment (start 98.5012 101.3319) (end 98.6645 101.3319) (width 0.127) (layer "F.Cu") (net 9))
 (segment (start 99.822 101.981) (end 100.137 101.666) (width 0.127) (layer "F.Cu") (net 9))
 (segment (start 98.6645 101.3319) (end 98.86 101.5274) (width 0.127) (layer "F.Cu") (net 9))
 (segment (start 98.86 101.5274) (end 98.86 101.8064) (width 0.127) (layer "F.Cu") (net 9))
 (segment (start 100.9535 101.6775) (end 100.965 101.666) (width 0.127) (layer "F.Cu") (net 9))
 (segment (start 100.137 101.666) (end 100.965 101.666) (width 0.127) (layer "F.Cu") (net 9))
 (segment (start 100.9535 104.0178) (end 100.9535 101.6775) (width 0.127) (layer "F.Cu") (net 9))
 (segment (start 98.86 101.8064) (end 99.0346 101.981) (width 0.127) (layer "F.Cu") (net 9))
 (segment (start 99.0346 101.981) (end 99.822 101.981) (width 0.127) (layer "F.Cu") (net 9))
 (segment (start 101.539 100.076) (end 101.727 100.076) (width 0.127) (layer "F.Cu") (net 12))
 (segment (start 101.646167 102.366633) (end 101.646167 104.0178) (width 0.127) (layer "F.Cu") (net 12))
 (segment (start 101.727 100.076) (end 102.1334 100.4824) (width 0.127) (layer "F.Cu") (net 12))
 (segment (start 102.1334 101.8794) (end 101.646167 102.366633) (width 0.127) (layer "F.Cu") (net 12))
 (segment (start 102.1334 100.4824) (end 102.1334 101.8794) (width 0.127) (layer "F.Cu") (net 12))
 (segment (start 101.299833 102.179567) (end 101.299833 103.8178) (width 0.127) (layer "F.Cu") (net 13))
 (segment (start 101.6762 101.666) (end 101.6762 101.8032) (width 0.127) (layer "F.Cu") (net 13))
 (segment (start 101.6762 101.8032) (end 101.299833 102.179567) (width 0.127) (layer "F.Cu") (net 13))
 (segment (start 100.9904 106.0958) (end 100.9904 105.6894) (width 0.127) (layer "F.Cu") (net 4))
 (segment (start 101.6 106.1974) (end 101.092 106.1974) (width 0.127) (layer "F.Cu") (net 4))
 (segment (start 101.5012 105.2548) (end 101.646167 105.109833) (width 0.127) (layer "F.Cu") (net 4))
 (segment (start 101.5012 106.0986) (end 101.5012 105.712) (width 0.127) (layer "F.Cu") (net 4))
 (segment (start 101.5012 105.362) (end 101.5012 105.2548) (width 0.127) (layer "F.Cu") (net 4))
 (segment (start 101.092 106.1974) (end 100.9904 106.0958) (width 0.127) (layer "F.Cu") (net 4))
 (segment (start 101.6 106.1974) (end 101.5012 106.0986) (width 0.127) (layer "F.Cu") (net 4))
 (segment (start 101.5012 105.712) (end 101.5012 105.362) (width 0.127) (layer "F.Cu") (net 4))
 (segment (start 101.646167 105.109833) (end 101.646167 104.8178) (width 0.127) (layer "F.Cu") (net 4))
 (via (at 100.9904 105.6894) (size 0.508) (drill 0.254) (layers "F.Cu" "B.Cu") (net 4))
 (via (at 93.8276 105.3084) (size 0.508) (drill 0.254) (layers "F.Cu" "B.Cu") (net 4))
 (segment (start 100.9904 105.6894) (end 100.9904 106.0196) (width 0.127) (layer "B.Cu") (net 4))
 (segment (start 100.9904 106.0196) (end 101.1682 106.1974) (width 0.127) (layer "B.Cu") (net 4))
 (segment (start 101.1682 106.1974) (end 101.6 106.1974) (width 0.127) (layer "B.Cu") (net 4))
 (segment (start 100.8126 105.1814) (end 93.9546 105.1814) (width 0.127) (layer "B.Cu") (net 4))
 (segment (start 100.9904 105.6894) (end 100.9904 105.3592) (width 0.127) (layer "B.Cu") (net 4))
 (segment (start 100.9904 105.3592) (end 100.8126 105.1814) (width 0.127) (layer "B.Cu") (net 4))
 (segment (start 93.9546 105.1814) (end 93.8276 105.3084) (width 0.127) (layer "B.Cu") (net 4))
 (segment (start 98.86 99.5394) (end 98.933 99.4664) (width 0.127) (layer "F.Cu") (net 1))
 (segment (start 99.6188 100.5409) (end 99.6188 100.9319) (width 0.127) (layer "F.Cu") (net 1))
 (segment (start 98.86 100.1046) (end 99.26 100.5046) (width 0.127) (layer "F.Cu") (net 1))
 (segment (start 100.6348 99.695) (end 102.0318 99.695) (width 0.127) (layer "F.Cu") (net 1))
 (segment (start 98.933 99.4664) (end 99.5934 99.4664) (width 0.127) (layer "F.Cu") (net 1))
 (segment (start 98.5012 100.1409) (end 98.6645 100.1409) (width 0.127) (layer "F.Cu") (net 1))
 (segment (start 102.4382 102.0064) (end 101.9925 102.4521) (width 0.127) (layer "F.Cu") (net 1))
 (segment (start 99.4233 100.7364) (end 99.6188 100.5409) (width 0.127) (layer "F.Cu") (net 1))
 (segment (start 98.6645 100.1409) (end 98.86 99.9454) (width 0.127) (layer "F.Cu") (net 1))
 (segment (start 102.0318 99.695) (end 102.4382 100.1014) (width 0.127) (layer "F.Cu") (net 1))
 (segment (start 99.4233 100.7364) (end 99.26 100.7364) (width 0.127) (layer "F.Cu") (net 1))
 (segment (start 99.5934 99.4664) (end 99.9744 99.8474) (width 0.127) (layer "F.Cu") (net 1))
 (segment (start 98.86 99.9454) (end 98.86 100.1046) (width 0.127) (layer "F.Cu") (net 1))
 (segment (start 99.9744 99.8474) (end 100.4824 99.8474) (width 0.127) (layer "F.Cu") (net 1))
 (segment (start 100.4824 99.8474) (end 100.6348 99.695) (width 0.127) (layer "F.Cu") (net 1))
 (segment (start 101.9925 102.4521) (end 101.9925 103.8178) (width 0.127) (layer "F.Cu") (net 1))
 (segment (start 98.86 99.9454) (end 98.86 99.5394) (width 0.127) (layer "F.Cu") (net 1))
 (segment (start 102.4382 100.1014) (end 102.4382 102.0064) (width 0.127) (layer "F.Cu") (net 1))
 (segment (start 99.6188 100.9319) (end 99.4233 100.7364) (width 0.127) (layer "F.Cu") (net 1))
 (segment (start 99.26 100.5046) (end 99.26 100.7364) (width 0.127) (layer "F.Cu") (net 1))
 (segment (start 100.9535 104.8178) (end 98.417 104.8178) (width 0.127) (layer "F.Cu") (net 5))
 (segment (start 98.417 104.8178) (end 96.3676 102.7684) (width 0.127) (layer "F.Cu") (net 5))
 (segment (start 100.9535 104.4178) (end 99.5156 104.4178) (width 0.127) (layer "F.Cu") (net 7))
 (segment (start 99.1362 104.0384) (end 98.7806 103.6828) (width 0.127) (layer "F.Cu") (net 7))
 (segment (start 99.5156 104.4178) (end 99.1362 104.0384) (width 0.127) (layer "F.Cu") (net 7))
 (via (at 96.3676 100.2284) (size 0.508) (drill 0.254) (layers "F.Cu" "B.Cu") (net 7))
 (via (at 98.7806 103.6828) (size 0.508) (drill 0.254) (layers "F.Cu" "B.Cu") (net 7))
 (segment (start 98.7298 103.632) (end 97.2058 103.632) (width 0.127) (layer "B.Cu") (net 7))
 (segment (start 98.7806 103.6828) (end 98.7298 103.632) (width 0.127) (layer "B.Cu") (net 7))
 (segment (start 97.2058 103.632) (end 96.3676 102.7938) (width 0.127) (layer "B.Cu") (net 7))
 (segment (start 96.3676 102.7938) (end 96.3676 100.2284) (width 0.127) (layer "B.Cu") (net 7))
 (segment (start 96.4692 105.2068) (end 96.3676 105.3084) (width 0.127) (layer "F.Cu") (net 3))
 (segment (start 101.299833 105.024367) (end 101.1174 105.2068) (width 0.127) (layer "F.Cu") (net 3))
 (segment (start 101.299833 104.6178) (end 101.299833 105.024367) (width 0.127) (layer "F.Cu") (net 3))
 (segment (start 101.1174 105.2068) (end 96.4692 105.2068) (width 0.127) (layer "F.Cu") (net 3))
 (segment (start 101.9925 105.2207) (end 101.8512 105.362) (width 0.127) (layer "F.Cu") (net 11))
 (segment (start 101.9925 104.6178) (end 101.9925 105.2207) (width 0.127) (layer "F.Cu") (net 11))
 (segment (start 100.7212 101.026) (end 99.8361 100.1409) (width 0.127) (layer "F.Cu") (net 15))
 (segment (start 99.8361 100.1409) (end 99.6188 100.1409) (width 0.127) (layer "F.Cu") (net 15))
 (segment (start 100.965 101.026) (end 100.7212 101.026) (width 0.127) (layer "F.Cu") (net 15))
 (segment (start 99.26 99.9454) (end 99.4555 100.1409) (width 0.127) (layer "F.Cu") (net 15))
 (segment (start 99.4555 100.1409) (end 99.6188 100.1409) (width 0.127) (layer "F.Cu") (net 15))
 (segment (start 100.899 100.3452) (end 100.8888 100.3554) (width 0.127) (layer "F.Cu") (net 2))
 (segment (start 100.899 100.076) (end 100.899 100.3452) (width 0.127) (layer "F.Cu") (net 2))
 (via (at 100.8888 100.3554) (size 0.508) (drill 0.254) (layers "F.Cu" "B.Cu") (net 2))
 (via (at 98.6536 100.7364) (size 0.508) (drill 0.254) (layers "F.Cu" "B.Cu") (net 2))
 (segment (start 100.8888 100.3554) (end 100.5078 100.7364) (width 0.127) (layer "B.Cu") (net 2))
 (segment (start 100.5078 100.7364) (end 98.6536 100.7364) (width 0.127) (layer "B.Cu") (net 2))
 (segment (start 101.6762 100.711) (end 101.6762 101.026) (width 0.127) (layer "F.Cu") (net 10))
 (segment (start 101.6508 100.6856) (end 101.6762 100.711) (width 0.127) (layer "F.Cu") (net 10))
 (via (at 99.5426 101.5238) (size 0.508) (drill 0.254) (layers "F.Cu" "B.Cu") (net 10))
 (via (at 101.6508 100.6856) (size 0.508) (drill 0.254) (layers "F.Cu" "B.Cu") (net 10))
 (segment (start 100.8126 101.5238) (end 99.5426 101.5238) (width 0.127) (layer "B.Cu") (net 10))
 (segment (start 101.6508 100.6856) (end 100.8126 101.5238) (width 0.127) (layer "B.Cu") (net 10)))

